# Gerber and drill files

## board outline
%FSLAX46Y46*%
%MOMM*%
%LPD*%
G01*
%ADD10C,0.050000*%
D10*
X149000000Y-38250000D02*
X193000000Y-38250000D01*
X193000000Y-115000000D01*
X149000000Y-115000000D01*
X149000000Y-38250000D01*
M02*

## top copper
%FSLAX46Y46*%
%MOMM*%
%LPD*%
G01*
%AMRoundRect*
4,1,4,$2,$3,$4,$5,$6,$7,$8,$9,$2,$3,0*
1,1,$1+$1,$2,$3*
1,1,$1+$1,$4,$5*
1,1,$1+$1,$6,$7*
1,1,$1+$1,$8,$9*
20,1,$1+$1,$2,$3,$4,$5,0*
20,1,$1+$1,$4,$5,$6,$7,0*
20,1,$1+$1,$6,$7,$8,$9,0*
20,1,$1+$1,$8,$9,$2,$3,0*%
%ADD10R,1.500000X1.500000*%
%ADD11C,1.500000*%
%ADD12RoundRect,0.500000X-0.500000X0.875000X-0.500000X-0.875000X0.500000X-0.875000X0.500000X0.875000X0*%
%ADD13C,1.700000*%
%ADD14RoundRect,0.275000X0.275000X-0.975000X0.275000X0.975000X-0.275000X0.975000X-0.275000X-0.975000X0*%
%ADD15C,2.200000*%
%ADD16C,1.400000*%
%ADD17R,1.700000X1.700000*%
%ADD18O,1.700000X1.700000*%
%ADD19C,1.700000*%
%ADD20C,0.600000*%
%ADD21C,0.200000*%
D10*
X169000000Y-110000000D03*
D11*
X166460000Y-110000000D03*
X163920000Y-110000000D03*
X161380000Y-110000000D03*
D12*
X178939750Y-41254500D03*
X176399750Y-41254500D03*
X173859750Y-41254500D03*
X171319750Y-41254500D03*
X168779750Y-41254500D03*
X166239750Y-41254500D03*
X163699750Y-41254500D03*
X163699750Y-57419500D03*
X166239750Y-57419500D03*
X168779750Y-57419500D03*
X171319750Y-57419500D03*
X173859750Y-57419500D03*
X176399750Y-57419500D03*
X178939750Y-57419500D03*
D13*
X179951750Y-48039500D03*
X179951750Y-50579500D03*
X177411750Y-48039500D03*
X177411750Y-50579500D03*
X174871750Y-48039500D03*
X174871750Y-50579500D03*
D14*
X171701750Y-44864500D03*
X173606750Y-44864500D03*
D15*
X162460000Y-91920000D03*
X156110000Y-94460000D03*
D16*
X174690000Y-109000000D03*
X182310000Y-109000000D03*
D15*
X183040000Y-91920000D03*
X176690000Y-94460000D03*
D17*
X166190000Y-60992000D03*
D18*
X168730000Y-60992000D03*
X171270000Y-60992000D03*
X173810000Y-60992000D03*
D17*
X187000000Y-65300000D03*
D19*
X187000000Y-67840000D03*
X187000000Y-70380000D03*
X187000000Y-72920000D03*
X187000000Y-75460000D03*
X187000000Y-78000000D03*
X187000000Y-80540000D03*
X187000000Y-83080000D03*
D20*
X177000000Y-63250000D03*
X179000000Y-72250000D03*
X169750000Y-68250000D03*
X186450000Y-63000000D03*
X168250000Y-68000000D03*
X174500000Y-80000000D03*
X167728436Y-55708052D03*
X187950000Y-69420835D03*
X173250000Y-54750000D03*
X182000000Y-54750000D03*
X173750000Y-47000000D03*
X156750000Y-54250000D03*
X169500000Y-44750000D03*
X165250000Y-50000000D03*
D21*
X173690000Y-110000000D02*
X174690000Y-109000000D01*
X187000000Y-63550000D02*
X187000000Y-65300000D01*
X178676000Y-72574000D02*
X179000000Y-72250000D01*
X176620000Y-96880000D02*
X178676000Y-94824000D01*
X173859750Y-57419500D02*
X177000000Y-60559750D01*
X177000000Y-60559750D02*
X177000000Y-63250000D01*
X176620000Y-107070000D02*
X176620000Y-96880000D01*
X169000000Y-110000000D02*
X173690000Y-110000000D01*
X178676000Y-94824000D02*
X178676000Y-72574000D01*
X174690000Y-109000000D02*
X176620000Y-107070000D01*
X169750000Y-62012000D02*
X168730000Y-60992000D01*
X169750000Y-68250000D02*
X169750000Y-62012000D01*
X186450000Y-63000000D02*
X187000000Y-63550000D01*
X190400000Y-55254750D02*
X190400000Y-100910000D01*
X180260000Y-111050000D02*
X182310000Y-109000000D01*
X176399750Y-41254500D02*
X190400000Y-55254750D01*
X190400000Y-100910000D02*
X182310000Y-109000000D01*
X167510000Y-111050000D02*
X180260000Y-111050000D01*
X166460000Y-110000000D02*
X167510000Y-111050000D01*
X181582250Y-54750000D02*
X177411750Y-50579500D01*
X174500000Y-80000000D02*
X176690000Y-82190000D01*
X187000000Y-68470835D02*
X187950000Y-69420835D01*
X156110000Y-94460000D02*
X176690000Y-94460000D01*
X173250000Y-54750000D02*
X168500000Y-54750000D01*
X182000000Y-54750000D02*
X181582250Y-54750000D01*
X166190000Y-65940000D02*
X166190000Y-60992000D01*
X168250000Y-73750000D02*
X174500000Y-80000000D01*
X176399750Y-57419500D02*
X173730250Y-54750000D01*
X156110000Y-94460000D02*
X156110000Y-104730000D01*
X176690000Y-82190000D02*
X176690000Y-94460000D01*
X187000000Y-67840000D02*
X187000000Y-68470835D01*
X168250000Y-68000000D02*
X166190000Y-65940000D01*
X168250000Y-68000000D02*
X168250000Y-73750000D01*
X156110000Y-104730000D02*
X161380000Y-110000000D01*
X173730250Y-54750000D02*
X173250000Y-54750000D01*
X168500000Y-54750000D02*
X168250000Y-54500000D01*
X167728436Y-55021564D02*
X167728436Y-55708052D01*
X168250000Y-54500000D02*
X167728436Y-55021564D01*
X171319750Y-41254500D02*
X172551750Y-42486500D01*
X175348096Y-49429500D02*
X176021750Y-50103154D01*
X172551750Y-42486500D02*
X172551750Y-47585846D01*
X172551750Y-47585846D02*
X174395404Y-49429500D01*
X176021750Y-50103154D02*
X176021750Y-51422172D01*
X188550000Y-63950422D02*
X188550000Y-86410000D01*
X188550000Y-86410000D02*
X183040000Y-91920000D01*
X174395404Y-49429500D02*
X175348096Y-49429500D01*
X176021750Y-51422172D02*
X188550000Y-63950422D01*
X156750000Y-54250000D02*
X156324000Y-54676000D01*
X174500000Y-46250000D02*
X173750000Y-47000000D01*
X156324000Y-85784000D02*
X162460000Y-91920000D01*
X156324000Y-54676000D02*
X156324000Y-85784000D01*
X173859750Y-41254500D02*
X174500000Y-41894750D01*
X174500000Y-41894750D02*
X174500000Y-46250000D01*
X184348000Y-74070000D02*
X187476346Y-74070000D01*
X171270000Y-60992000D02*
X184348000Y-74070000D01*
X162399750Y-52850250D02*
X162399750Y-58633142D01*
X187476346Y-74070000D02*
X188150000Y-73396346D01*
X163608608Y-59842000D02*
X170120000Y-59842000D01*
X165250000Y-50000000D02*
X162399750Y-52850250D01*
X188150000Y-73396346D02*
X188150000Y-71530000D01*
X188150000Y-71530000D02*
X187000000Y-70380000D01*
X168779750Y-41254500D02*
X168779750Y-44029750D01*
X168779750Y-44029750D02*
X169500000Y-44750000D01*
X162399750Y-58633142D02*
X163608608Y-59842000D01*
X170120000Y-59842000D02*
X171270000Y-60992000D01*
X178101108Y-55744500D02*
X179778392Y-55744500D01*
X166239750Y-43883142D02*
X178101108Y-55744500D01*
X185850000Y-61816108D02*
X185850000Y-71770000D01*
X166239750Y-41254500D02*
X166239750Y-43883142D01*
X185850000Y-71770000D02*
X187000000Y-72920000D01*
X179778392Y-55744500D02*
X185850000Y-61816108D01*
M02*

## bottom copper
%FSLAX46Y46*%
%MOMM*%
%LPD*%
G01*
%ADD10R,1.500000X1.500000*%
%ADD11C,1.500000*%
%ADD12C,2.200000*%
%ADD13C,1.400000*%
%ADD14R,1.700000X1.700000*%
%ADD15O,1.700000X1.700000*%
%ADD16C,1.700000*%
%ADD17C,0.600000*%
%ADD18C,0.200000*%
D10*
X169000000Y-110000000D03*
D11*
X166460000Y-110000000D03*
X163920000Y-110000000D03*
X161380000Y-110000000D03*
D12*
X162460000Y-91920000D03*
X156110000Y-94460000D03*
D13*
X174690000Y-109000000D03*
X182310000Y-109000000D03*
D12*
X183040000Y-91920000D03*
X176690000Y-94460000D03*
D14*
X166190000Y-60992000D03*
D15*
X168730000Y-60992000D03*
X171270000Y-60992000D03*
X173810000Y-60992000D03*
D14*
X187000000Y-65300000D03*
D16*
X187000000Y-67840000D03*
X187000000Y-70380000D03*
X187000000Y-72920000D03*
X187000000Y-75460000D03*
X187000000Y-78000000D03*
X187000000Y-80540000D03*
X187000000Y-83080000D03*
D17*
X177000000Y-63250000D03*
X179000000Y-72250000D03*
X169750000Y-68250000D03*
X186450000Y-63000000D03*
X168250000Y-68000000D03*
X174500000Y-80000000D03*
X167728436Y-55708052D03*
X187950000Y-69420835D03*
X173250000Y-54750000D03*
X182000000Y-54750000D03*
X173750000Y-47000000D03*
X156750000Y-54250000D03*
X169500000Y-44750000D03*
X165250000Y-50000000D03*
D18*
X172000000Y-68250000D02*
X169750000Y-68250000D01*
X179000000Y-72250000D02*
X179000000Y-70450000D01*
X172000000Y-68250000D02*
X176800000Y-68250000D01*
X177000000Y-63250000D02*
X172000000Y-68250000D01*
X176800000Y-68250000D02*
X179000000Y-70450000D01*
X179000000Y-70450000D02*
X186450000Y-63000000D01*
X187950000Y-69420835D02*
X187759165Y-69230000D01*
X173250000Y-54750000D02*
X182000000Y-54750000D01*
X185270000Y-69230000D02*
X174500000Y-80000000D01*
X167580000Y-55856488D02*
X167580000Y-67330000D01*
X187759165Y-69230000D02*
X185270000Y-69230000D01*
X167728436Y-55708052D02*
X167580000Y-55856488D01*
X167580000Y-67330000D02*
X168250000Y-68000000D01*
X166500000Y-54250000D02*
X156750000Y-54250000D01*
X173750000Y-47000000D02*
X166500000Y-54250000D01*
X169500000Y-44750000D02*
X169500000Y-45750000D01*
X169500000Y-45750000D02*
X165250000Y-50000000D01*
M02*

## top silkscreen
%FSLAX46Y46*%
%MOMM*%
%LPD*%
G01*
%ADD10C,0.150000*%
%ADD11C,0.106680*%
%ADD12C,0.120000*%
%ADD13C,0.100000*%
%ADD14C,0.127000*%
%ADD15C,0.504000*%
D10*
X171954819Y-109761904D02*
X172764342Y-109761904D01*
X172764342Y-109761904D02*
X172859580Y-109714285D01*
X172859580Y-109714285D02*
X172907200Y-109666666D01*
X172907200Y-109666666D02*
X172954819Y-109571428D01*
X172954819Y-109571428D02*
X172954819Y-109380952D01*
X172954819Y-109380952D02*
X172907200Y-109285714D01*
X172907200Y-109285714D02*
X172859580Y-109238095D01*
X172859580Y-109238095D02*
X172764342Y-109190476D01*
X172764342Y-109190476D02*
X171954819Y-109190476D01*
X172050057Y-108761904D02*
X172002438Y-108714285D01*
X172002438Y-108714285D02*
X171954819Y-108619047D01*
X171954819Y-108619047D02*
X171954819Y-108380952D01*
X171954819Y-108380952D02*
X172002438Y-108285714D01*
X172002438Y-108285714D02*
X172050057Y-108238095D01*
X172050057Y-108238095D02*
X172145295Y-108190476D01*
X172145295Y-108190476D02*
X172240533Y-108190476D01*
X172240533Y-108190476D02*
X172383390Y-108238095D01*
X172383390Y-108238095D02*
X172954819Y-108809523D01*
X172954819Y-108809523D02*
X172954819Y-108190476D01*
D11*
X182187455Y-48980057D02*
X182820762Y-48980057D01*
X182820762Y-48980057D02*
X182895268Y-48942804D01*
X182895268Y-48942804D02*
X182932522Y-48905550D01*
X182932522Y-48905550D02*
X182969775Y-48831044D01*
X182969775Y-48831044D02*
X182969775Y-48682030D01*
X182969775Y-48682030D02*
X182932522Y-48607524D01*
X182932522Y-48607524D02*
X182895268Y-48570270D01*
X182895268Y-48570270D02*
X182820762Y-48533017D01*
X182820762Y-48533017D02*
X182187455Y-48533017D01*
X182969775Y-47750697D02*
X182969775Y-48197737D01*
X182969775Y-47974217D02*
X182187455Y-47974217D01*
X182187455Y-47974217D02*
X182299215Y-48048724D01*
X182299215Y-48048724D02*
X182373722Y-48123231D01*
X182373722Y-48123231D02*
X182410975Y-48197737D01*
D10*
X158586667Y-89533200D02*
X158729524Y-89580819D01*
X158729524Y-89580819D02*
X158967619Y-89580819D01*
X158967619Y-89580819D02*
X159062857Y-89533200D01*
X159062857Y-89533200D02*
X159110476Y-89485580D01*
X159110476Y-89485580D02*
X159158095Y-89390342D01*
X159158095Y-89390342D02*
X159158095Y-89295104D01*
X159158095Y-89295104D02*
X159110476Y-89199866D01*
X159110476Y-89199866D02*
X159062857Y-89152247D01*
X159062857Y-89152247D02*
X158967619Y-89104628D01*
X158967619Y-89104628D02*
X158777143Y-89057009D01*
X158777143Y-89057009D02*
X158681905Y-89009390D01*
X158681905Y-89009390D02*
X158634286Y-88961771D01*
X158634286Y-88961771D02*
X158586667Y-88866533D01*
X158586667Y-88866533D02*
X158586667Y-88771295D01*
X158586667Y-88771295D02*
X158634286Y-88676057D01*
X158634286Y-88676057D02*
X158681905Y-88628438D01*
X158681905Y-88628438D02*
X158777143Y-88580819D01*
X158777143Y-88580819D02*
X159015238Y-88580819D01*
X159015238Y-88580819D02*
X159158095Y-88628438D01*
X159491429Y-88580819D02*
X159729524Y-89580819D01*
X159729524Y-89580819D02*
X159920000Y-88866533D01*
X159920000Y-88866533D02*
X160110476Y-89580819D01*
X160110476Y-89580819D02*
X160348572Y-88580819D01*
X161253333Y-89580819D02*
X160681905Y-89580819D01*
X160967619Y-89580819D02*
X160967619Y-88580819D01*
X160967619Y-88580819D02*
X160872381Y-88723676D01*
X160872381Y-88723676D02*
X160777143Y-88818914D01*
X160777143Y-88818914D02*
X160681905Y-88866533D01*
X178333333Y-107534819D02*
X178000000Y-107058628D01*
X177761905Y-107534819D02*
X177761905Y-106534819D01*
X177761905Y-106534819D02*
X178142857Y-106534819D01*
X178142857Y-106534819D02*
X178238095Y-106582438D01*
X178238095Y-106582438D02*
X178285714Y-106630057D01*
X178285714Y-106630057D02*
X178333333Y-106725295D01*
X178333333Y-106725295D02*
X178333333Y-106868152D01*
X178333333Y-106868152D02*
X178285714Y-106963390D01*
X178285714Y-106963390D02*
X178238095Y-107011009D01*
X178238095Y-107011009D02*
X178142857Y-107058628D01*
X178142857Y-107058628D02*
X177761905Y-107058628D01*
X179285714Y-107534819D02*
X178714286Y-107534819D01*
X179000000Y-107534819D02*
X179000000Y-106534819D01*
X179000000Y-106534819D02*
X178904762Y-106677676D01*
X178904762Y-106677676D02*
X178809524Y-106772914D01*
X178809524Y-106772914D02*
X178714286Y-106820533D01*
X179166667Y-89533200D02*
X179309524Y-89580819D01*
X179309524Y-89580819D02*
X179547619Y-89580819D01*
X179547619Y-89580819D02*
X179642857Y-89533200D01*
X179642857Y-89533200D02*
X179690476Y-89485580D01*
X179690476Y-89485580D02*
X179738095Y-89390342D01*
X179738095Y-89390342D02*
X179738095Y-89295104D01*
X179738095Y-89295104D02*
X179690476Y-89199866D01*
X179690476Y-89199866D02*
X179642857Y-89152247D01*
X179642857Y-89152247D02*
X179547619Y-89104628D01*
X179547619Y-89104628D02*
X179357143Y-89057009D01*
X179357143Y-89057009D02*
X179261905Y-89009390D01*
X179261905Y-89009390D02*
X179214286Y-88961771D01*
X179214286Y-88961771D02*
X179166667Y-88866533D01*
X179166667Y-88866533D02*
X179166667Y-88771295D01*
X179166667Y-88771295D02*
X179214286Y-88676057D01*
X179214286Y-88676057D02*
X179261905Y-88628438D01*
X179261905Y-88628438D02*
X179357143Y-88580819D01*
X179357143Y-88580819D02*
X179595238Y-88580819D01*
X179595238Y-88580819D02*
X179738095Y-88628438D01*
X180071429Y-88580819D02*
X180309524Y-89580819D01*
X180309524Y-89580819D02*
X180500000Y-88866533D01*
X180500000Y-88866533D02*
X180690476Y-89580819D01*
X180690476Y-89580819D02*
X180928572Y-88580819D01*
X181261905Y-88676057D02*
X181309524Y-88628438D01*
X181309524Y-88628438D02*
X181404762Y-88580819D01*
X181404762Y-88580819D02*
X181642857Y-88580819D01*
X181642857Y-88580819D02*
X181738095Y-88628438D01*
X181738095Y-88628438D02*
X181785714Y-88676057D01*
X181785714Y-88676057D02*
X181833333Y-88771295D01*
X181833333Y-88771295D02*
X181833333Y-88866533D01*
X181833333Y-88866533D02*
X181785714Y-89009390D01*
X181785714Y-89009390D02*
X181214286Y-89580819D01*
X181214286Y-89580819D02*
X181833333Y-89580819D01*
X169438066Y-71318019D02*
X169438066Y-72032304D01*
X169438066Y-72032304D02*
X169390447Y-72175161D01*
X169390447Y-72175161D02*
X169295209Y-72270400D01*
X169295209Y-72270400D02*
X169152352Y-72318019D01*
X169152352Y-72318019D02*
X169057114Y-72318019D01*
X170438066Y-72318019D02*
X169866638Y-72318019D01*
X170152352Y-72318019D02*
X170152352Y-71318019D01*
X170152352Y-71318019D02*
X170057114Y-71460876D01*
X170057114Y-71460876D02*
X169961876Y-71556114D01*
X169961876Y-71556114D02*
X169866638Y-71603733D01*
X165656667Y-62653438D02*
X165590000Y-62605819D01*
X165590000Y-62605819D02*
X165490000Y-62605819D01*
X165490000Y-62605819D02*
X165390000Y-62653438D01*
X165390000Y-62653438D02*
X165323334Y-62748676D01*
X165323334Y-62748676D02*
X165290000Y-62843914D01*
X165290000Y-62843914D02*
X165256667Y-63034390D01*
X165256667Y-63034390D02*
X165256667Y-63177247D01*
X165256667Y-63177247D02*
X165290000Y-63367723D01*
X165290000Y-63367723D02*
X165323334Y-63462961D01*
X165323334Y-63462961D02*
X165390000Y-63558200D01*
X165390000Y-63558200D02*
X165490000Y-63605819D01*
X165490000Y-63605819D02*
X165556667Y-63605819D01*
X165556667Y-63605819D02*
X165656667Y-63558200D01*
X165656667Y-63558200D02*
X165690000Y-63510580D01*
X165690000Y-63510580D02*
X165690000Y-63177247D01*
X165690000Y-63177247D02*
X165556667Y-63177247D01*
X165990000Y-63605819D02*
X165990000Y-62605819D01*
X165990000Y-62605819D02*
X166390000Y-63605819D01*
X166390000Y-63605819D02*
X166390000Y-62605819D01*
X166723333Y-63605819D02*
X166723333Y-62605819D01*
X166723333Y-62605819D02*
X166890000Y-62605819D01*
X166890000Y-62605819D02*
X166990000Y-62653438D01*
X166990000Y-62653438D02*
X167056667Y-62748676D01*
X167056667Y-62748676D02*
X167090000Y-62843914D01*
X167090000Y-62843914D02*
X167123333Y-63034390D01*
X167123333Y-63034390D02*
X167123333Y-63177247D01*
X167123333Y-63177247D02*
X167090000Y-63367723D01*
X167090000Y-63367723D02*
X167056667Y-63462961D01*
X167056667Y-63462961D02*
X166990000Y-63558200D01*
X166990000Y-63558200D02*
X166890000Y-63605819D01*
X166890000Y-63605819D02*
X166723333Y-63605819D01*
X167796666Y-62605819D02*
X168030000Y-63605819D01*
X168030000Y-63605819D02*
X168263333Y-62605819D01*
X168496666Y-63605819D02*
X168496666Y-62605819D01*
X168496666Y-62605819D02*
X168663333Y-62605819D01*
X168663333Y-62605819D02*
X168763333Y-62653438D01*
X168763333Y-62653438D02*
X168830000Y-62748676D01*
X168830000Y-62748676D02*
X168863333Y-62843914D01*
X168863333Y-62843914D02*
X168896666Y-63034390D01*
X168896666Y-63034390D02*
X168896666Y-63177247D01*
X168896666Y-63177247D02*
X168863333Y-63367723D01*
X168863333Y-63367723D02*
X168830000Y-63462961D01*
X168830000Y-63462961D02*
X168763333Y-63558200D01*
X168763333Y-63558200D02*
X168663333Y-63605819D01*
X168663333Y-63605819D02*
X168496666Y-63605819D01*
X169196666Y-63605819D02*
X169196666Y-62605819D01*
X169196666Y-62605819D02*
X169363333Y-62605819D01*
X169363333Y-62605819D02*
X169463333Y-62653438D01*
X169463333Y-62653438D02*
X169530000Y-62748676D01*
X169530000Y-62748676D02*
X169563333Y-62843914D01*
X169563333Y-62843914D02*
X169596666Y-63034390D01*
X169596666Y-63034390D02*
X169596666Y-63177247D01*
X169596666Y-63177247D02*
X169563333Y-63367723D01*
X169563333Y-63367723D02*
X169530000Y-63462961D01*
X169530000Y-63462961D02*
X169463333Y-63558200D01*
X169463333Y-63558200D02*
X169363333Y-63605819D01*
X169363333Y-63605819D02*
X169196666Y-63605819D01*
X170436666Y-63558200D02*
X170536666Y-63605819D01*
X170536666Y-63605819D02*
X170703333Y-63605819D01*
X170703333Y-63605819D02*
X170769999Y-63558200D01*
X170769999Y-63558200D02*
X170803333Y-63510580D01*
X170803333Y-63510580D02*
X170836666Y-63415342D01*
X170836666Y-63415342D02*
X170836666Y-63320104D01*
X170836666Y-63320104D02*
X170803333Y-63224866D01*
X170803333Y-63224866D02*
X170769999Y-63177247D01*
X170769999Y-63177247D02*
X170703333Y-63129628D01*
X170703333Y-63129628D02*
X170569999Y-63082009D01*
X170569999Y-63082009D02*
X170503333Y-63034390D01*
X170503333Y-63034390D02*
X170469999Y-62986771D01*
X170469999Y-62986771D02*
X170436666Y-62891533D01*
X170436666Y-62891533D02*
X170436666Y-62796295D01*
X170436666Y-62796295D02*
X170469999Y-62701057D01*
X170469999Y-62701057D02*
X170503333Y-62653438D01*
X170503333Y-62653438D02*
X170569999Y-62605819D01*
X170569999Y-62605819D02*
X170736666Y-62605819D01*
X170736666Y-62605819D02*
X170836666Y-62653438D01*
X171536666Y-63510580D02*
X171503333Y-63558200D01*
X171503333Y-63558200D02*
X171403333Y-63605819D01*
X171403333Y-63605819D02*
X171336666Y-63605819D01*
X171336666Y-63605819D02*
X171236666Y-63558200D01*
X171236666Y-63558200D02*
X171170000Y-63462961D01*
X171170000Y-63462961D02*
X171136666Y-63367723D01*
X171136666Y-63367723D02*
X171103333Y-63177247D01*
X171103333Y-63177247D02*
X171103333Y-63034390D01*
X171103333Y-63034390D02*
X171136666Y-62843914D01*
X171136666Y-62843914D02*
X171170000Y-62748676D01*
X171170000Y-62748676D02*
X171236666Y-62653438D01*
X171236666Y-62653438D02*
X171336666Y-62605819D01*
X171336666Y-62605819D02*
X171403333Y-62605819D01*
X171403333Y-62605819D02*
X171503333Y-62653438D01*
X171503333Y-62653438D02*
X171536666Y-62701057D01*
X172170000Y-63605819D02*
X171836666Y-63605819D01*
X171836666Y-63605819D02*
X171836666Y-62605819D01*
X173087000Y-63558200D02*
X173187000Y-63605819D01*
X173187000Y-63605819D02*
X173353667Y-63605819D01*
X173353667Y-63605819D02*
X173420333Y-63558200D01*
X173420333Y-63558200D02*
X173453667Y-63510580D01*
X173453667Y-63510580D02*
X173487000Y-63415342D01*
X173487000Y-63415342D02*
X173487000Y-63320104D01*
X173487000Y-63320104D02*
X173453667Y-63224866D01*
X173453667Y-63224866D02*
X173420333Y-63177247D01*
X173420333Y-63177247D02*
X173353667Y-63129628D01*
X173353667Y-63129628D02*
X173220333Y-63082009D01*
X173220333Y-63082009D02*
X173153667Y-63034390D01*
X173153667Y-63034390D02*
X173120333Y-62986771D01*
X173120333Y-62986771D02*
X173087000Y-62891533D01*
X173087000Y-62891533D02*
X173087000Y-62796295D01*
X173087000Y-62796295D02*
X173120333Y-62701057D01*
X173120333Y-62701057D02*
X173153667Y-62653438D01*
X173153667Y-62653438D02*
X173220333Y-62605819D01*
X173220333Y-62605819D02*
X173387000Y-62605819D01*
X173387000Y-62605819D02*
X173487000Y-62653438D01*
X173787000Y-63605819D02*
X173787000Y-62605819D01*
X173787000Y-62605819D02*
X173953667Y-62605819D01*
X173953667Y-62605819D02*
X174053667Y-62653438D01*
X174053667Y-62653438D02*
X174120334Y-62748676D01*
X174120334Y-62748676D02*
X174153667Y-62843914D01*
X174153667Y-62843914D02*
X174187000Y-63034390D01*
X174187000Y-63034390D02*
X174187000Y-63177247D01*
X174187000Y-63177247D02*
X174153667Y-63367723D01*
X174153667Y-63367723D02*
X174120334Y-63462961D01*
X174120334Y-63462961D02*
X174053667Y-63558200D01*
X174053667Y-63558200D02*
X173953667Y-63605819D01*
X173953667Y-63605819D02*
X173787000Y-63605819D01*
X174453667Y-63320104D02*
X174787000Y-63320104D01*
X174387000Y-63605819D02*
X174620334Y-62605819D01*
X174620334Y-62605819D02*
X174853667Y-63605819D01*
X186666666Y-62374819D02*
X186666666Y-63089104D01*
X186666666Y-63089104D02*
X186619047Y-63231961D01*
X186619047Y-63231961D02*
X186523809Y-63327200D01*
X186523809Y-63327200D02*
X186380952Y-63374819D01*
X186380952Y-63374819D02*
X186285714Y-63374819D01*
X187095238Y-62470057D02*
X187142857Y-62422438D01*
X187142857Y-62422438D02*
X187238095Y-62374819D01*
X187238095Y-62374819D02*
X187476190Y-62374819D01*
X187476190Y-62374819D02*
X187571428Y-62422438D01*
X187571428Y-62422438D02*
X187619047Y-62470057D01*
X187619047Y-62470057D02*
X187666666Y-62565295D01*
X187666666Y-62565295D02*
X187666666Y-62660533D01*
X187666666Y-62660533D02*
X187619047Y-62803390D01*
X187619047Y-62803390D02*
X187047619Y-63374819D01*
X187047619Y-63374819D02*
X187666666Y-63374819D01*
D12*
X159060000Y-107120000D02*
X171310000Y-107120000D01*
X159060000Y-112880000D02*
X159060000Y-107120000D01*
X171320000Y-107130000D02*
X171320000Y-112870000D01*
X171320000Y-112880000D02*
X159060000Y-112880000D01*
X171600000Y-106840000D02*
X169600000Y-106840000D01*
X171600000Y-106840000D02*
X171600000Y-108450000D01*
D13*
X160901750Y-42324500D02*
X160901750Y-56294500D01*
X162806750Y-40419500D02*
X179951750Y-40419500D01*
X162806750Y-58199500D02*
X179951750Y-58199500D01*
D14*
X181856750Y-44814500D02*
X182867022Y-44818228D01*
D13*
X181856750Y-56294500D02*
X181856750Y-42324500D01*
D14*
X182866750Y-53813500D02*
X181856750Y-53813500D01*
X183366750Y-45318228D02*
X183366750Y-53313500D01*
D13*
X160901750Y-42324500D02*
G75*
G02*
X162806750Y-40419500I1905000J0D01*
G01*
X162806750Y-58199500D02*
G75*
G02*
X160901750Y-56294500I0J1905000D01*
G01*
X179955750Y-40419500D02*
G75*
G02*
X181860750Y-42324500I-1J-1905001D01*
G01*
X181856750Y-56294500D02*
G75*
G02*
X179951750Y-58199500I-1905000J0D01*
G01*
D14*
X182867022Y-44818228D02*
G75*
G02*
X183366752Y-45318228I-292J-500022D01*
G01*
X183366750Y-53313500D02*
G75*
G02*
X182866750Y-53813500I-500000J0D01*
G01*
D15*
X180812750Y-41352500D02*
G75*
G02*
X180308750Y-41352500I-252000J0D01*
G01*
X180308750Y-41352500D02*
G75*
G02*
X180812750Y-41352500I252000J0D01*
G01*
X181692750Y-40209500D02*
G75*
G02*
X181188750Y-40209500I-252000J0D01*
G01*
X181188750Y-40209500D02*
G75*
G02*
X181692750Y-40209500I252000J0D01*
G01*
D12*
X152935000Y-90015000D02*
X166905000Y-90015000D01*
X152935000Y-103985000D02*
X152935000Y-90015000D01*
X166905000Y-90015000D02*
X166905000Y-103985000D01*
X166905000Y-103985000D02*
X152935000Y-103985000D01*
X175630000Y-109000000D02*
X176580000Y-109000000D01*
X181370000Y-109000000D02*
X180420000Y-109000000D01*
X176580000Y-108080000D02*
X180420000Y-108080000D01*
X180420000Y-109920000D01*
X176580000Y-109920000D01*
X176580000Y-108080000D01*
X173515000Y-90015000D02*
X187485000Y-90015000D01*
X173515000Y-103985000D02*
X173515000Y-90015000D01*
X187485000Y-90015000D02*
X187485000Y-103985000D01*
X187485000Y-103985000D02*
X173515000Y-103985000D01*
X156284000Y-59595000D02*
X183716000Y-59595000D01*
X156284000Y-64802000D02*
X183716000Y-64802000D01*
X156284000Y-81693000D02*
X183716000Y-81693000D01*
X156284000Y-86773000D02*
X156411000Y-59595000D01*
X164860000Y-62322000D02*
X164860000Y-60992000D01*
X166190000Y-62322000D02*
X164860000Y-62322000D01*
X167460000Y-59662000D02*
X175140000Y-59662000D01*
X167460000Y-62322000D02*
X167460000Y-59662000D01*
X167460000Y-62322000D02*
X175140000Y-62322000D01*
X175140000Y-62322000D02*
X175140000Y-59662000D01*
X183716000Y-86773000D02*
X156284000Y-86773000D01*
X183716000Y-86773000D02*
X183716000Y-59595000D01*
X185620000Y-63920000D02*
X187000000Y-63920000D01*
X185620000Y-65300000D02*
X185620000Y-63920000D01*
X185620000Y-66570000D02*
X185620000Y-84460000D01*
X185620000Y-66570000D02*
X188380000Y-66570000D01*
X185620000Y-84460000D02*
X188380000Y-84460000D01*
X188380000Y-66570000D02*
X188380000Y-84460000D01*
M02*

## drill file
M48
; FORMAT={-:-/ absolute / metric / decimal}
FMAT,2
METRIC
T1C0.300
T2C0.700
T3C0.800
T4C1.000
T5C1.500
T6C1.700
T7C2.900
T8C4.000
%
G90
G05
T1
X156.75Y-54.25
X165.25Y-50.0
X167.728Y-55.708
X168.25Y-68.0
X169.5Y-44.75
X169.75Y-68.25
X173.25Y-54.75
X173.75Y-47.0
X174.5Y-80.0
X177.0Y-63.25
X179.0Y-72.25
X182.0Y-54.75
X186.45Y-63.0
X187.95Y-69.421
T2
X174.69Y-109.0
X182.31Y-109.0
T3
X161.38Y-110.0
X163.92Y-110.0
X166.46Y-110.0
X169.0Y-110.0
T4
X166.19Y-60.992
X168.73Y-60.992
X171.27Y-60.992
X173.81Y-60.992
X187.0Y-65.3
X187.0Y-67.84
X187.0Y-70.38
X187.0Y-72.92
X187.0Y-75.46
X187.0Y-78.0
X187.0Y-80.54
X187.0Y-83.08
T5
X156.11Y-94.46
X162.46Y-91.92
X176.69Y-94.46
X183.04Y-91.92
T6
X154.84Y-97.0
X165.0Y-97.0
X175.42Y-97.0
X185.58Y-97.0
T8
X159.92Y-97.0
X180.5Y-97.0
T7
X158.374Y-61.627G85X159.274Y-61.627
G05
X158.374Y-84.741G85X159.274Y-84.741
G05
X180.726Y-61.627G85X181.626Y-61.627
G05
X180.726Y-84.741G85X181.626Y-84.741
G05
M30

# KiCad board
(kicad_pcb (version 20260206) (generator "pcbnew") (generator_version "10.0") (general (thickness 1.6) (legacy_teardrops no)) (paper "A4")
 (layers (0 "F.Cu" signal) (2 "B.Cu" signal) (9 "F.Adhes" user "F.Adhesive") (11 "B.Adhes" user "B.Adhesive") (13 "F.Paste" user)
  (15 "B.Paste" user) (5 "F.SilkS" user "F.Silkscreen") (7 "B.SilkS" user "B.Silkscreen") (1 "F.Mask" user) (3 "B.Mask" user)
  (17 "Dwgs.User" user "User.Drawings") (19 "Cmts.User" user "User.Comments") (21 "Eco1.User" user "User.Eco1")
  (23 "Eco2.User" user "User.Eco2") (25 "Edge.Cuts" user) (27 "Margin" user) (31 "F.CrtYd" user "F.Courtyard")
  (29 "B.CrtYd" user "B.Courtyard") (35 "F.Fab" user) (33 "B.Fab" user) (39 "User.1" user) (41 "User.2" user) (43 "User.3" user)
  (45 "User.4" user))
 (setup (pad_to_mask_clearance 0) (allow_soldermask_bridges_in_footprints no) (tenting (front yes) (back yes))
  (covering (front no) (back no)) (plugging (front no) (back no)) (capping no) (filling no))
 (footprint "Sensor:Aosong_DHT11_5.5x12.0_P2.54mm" (layer "F.Cu") (at 169 110 -90)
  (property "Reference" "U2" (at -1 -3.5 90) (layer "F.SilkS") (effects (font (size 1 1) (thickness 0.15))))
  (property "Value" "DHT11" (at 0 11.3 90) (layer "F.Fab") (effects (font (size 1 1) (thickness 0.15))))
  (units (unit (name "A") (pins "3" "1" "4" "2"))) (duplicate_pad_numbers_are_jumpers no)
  (fp_line (start -2.88 9.94) (end -2.88 -2.31) (stroke (width 0.12) (type solid)) (layer "F.SilkS"))
  (fp_line (start 2.88 9.94) (end -2.88 9.94) (stroke (width 0.12) (type solid)) (layer "F.SilkS"))
  (fp_line (start -2.87 -2.32) (end 2.87 -2.32) (stroke (width 0.12) (type solid)) (layer "F.SilkS"))
  (fp_line (start 2.88 -2.32) (end 2.88 9.94) (stroke (width 0.12) (type solid)) (layer "F.SilkS"))
  (fp_line (start -3.16 -2.6) (end -3.16 -0.6) (stroke (width 0.12) (type solid)) (layer "F.SilkS"))
  (fp_line (start -3.16 -2.6) (end -1.55 -2.6) (stroke (width 0.12) (type solid)) (layer "F.SilkS"))
  (pad "1" thru_hole rect (at 0 0 270) (size 1.5 1.5) (drill 0.8) (layers "*.Cu" "*.Mask") (remove_unused_layers no) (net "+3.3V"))
  (pad "2" thru_hole circle (at 0 2.54 270) (size 1.5 1.5) (drill 0.8) (layers "*.Cu" "*.Mask") (remove_unused_layers no)
   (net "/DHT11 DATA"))
  (pad "3" thru_hole circle (at 0 5.08 270) (size 1.5 1.5) (drill 0.8) (layers "*.Cu" "*.Mask") (remove_unused_layers no)
   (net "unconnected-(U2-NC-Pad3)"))
  (pad "4" thru_hole circle (at 0 7.62 270) (size 1.5 1.5) (drill 0.8) (layers "*.Cu" "*.Mask") (remove_unused_layers no) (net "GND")))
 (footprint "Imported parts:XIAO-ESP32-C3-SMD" (layer "F.Cu") (at 160.81975 40.4195 -90)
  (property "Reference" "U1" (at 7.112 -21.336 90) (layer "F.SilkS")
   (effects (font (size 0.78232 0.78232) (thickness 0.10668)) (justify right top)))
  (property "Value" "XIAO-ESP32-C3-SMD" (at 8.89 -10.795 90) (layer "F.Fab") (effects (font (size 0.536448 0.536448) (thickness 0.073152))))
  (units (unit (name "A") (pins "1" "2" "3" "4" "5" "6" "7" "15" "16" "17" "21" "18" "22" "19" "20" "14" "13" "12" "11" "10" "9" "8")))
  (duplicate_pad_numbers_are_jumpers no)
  (fp_line (start 1.905 -0.082) (end 15.875 -0.082) (stroke (width 0.1) (type solid)) (layer "F.SilkS"))
  (fp_line (start 0 -1.987) (end 0 -19.132) (stroke (width 0.1) (type solid)) (layer "F.SilkS"))
  (fp_line (start 17.78 -1.987) (end 17.78 -19.132) (stroke (width 0.1) (type solid)) (layer "F.SilkS"))
  (fp_line (start 4.395 -21.037) (end 4.398728 -22.047272) (stroke (width 0.127) (type solid)) (layer "F.SilkS"))
  (fp_line (start 15.875 -21.037) (end 1.905 -21.037) (stroke (width 0.1) (type solid)) (layer "F.SilkS"))
  (fp_line (start 13.394 -22.047) (end 13.394 -21.037) (stroke (width 0.127) (type solid)) (layer "F.SilkS"))
  (fp_line (start 4.898728 -22.547) (end 12.894 -22.547) (stroke (width 0.127) (type solid)) (layer "F.SilkS"))
  (fp_arc (start 1.905 -0.082) (mid 0.557962 -0.639962) (end 0 -1.987) (stroke (width 0.1) (type solid)) (layer "F.SilkS"))
  (fp_arc (start 17.78 -1.987) (mid 17.222038 -0.639962) (end 15.875 -0.082) (stroke (width 0.1) (type solid)) (layer "F.SilkS"))
  (fp_arc (start 0 -19.136) (mid 0.557962 -20.483038) (end 1.905 -21.041) (stroke (width 0.1) (type solid)) (layer "F.SilkS"))
  (fp_arc (start 15.875 -21.037) (mid 17.222038 -20.479038) (end 17.78 -19.132) (stroke (width 0.1) (type solid)) (layer "F.SilkS"))
  (fp_arc (start 4.398728 -22.047272) (mid 4.545272 -22.40064) (end 4.898728 -22.547) (stroke (width 0.127) (type default))
   (layer "F.SilkS"))
  (fp_arc (start 12.894 -22.547) (mid 13.247553 -22.400553) (end 13.394 -22.047) (stroke (width 0.127) (type default)) (layer "F.SilkS"))
  (fp_circle (center 0.933 -19.741) (end 0.933 -19.995) (stroke (width 0.5) (type solid)) (fill yes) (layer "F.SilkS"))
  (fp_circle (center -0.21 -20.621) (end -0.21 -20.875) (stroke (width 0.5) (type solid)) (fill yes) (layer "F.SilkS"))
  (pad "1" smd roundrect (at 0.835 -18.12 270) (size 2.75 2) (layers "F.Cu" "F.Mask" "F.Paste") (roundrect_rratio 0.25)
   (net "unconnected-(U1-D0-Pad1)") (solder_mask_margin 0.0508) (thermal_bridge_angle 45))
  (pad "2" smd roundrect (at 0.835 -15.58 270) (size 2.75 2) (layers "F.Cu" "F.Mask" "F.Paste") (roundrect_rratio 0.25) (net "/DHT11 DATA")
   (solder_mask_margin 0.0508) (thermal_bridge_angle 45))
  (pad "3" smd roundrect (at 0.835 -13.04 270) (size 2.75 2) (layers "F.Cu" "F.Mask" "F.Paste") (roundrect_rratio 0.25) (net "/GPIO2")
   (solder_mask_margin 0.0508) (thermal_bridge_angle 45))
  (pad "4" smd roundrect (at 0.835 -10.5 270) (size 2.75 2) (layers "F.Cu" "F.Mask" "F.Paste") (roundrect_rratio 0.25) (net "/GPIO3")
   (solder_mask_margin 0.0508) (thermal_bridge_angle 45))
  (pad "5" smd roundrect (at 0.835 -7.96 270) (size 2.75 2) (layers "F.Cu" "F.Mask" "F.Paste") (roundrect_rratio 0.25) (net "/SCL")
   (solder_mask_margin 0.0508) (thermal_bridge_angle 45))
  (pad "6" smd roundrect (at 0.835 -5.42 270) (size 2.75 2) (layers "F.Cu" "F.Mask" "F.Paste") (roundrect_rratio 0.25) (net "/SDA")
   (solder_mask_margin 0.0508) (thermal_bridge_angle 45))
  (pad "7" smd roundrect (at 0.835 -2.88 270) (size 2.75 2) (layers "F.Cu" "F.Mask" "F.Paste") (roundrect_rratio 0.25)
   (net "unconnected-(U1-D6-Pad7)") (solder_mask_margin 0.0508) (thermal_bridge_angle 45))
  (pad "8" smd roundrect (at 17 -2.88 270) (size 2.75 2) (layers "F.Cu" "F.Mask" "F.Paste") (roundrect_rratio 0.25)
   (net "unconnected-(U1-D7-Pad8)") (solder_mask_margin 0.0508) (thermal_bridge_angle 45))
  (pad "9" smd roundrect (at 17 -5.42 270) (size 2.75 2) (layers "F.Cu" "F.Mask" "F.Paste") (roundrect_rratio 0.25)
   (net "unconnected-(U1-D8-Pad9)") (solder_mask_margin 0.0508) (thermal_bridge_angle 45))
  (pad "10" smd roundrect (at 17 -7.96 270) (size 2.75 2) (layers "F.Cu" "F.Mask" "F.Paste") (roundrect_rratio 0.25)
   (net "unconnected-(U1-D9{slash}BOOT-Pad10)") (solder_mask_margin 0.0508) (thermal_bridge_angle 45))
  (pad "11" smd roundrect (at 17 -10.5 270) (size 2.75 2) (layers "F.Cu" "F.Mask" "F.Paste") (roundrect_rratio 0.25)
   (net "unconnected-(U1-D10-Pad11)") (solder_mask_margin 0.0508) (thermal_bridge_angle 45))
  (pad "12" smd roundrect (at 17 -13.04 270) (size 2.75 2) (layers "F.Cu" "F.Mask" "F.Paste") (roundrect_rratio 0.25) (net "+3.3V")
   (solder_mask_margin 0.0508) (thermal_bridge_angle 45))
  (pad "13" smd roundrect (at 17 -15.58 270) (size 2.75 2) (layers "F.Cu" "F.Mask" "F.Paste") (roundrect_rratio 0.25) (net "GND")
   (solder_mask_margin 0.0508) (thermal_bridge_angle 45))
  (pad "14" smd roundrect (at 17 -18.12 270) (size 2.75 2) (layers "F.Cu" "F.Mask" "F.Paste") (roundrect_rratio 0.25) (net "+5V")
   (solder_mask_margin 0.0508) (thermal_bridge_angle 45))
  (pad "15" smd circle (at 7.62 -19.132 270) (size 1.7 1.7) (layers "F.Cu" "F.Mask" "F.Paste") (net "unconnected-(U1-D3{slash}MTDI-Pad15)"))
  (pad "16" smd circle (at 10.16 -19.132 270) (size 1.7 1.7) (layers "F.Cu" "F.Mask" "F.Paste") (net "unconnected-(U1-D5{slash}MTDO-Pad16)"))
  (pad "17" smd circle (at 7.62 -16.592 270) (size 1.7 1.7) (layers "F.Cu" "F.Mask" "F.Paste") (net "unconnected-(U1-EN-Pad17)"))
  (pad "18" smd circle (at 10.16 -16.592 270) (size 1.7 1.7) (layers "F.Cu" "F.Mask" "F.Paste") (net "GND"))
  (pad "19" smd circle (at 7.62 -14.052 270) (size 1.7 1.7) (layers "F.Cu" "F.Mask" "F.Paste") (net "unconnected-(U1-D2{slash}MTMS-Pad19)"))
  (pad "20" smd circle (at 10.16 -14.052 270) (size 1.7 1.7) (layers "F.Cu" "F.Mask" "F.Paste") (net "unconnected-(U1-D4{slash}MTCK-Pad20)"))
  (pad "21" smd roundrect (at 4.445 -10.882 90) (size 2.5 1.1) (layers "F.Cu" "F.Mask" "F.Paste") (roundrect_rratio 0.25)
   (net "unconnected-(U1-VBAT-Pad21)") (thermal_bridge_angle 45))
  (pad "22" smd roundrect (at 4.445 -12.787 90) (size 2.5 1.1) (layers "F.Cu" "F.Mask" "F.Paste") (roundrect_rratio 0.25)
   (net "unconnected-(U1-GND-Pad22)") (thermal_bridge_angle 45)))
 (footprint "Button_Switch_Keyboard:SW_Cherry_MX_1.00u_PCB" (layer "F.Cu") (at 162.46 91.92)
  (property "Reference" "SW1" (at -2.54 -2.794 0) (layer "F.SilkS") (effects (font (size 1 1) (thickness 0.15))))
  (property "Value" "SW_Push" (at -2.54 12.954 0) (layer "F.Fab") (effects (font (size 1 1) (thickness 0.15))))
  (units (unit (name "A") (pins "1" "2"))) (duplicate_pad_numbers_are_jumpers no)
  (fp_line (start -9.525 -1.905) (end 4.445 -1.905) (stroke (width 0.12) (type solid)) (layer "F.SilkS"))
  (fp_line (start -9.525 12.065) (end -9.525 -1.905) (stroke (width 0.12) (type solid)) (layer "F.SilkS"))
  (fp_line (start 4.445 -1.905) (end 4.445 12.065) (stroke (width 0.12) (type solid)) (layer "F.SilkS"))
  (fp_line (start 4.445 12.065) (end -9.525 12.065) (stroke (width 0.12) (type solid)) (layer "F.SilkS"))
  (pad "" np_thru_hole circle (at -7.62 5.08) (size 1.7 1.7) (drill 1.7) (layers "*.Cu" "*.Mask"))
  (pad "" np_thru_hole circle (at -2.54 5.08) (size 4 4) (drill 4) (layers "*.Cu" "*.Mask"))
  (pad "" np_thru_hole circle (at 2.54 5.08) (size 1.7 1.7) (drill 1.7) (layers "*.Cu" "*.Mask"))
  (pad "1" thru_hole circle (at 0 0) (size 2.2 2.2) (drill 1.5) (layers "*.Cu" "*.Mask") (remove_unused_layers no) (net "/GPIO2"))
  (pad "2" thru_hole circle (at -6.35 2.54) (size 2.2 2.2) (drill 1.5) (layers "*.Cu" "*.Mask") (remove_unused_layers no) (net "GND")))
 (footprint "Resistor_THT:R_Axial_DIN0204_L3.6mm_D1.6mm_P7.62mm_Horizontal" (layer "F.Cu") (at 174.69 109)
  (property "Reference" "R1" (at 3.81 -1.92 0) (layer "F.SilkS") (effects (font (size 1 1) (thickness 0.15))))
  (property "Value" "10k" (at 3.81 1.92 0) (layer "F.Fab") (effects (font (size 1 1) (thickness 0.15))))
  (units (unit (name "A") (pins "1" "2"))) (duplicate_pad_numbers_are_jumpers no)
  (fp_line (start 0.94 0) (end 1.89 0) (stroke (width 0.12) (type solid)) (layer "F.SilkS"))
  (fp_line (start 6.68 0) (end 5.73 0) (stroke (width 0.12) (type solid)) (layer "F.SilkS"))
  (fp_rect (start 1.89 -0.92) (end 5.73 0.92) (stroke (width 0.12) (type solid)) (fill no) (layer "F.SilkS"))
  (pad "1" thru_hole circle (at 0 0) (size 1.4 1.4) (drill 0.7) (layers "*.Cu" "*.Mask") (remove_unused_layers no) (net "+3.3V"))
  (pad "2" thru_hole circle (at 7.62 0) (size 1.4 1.4) (drill 0.7) (layers "*.Cu" "*.Mask") (remove_unused_layers no) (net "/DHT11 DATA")))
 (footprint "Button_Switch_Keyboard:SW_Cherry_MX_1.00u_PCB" (layer "F.Cu") (at 183.04 91.92)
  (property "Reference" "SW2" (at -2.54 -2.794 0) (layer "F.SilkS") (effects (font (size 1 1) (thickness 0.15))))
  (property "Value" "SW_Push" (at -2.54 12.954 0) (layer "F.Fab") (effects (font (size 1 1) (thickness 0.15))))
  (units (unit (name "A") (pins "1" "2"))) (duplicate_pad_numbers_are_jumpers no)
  (fp_line (start -9.525 -1.905) (end 4.445 -1.905) (stroke (width 0.12) (type solid)) (layer "F.SilkS"))
  (fp_line (start -9.525 12.065) (end -9.525 -1.905) (stroke (width 0.12) (type solid)) (layer "F.SilkS"))
  (fp_line (start 4.445 -1.905) (end 4.445 12.065) (stroke (width 0.12) (type solid)) (layer "F.SilkS"))
  (fp_line (start 4.445 12.065) (end -9.525 12.065) (stroke (width 0.12) (type solid)) (layer "F.SilkS"))
  (pad "" np_thru_hole circle (at -7.62 5.08) (size 1.7 1.7) (drill 1.7) (layers "*.Cu" "*.Mask"))
  (pad "" np_thru_hole circle (at -2.54 5.08) (size 4 4) (drill 4) (layers "*.Cu" "*.Mask"))
  (pad "" np_thru_hole circle (at 2.54 5.08) (size 1.7 1.7) (drill 1.7) (layers "*.Cu" "*.Mask"))
  (pad "1" thru_hole circle (at 0 0) (size 2.2 2.2) (drill 1.5) (layers "*.Cu" "*.Mask") (remove_unused_layers no) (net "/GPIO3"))
  (pad "2" thru_hole circle (at -6.35 2.54) (size 2.2 2.2) (drill 1.5) (layers "*.Cu" "*.Mask") (remove_unused_layers no) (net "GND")))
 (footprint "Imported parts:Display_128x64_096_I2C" (layer "F.Cu") (at 170 60.992)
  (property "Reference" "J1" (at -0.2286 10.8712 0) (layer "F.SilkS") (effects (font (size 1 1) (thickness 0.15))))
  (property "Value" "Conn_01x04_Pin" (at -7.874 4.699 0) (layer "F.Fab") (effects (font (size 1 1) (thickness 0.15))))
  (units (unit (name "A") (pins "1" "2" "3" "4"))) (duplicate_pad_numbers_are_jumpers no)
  (fp_line (start -13.716 -1.397) (end 13.716 -1.397) (stroke (width 0.12) (type solid)) (layer "F.SilkS"))
  (fp_line (start -13.716 3.81) (end 13.716 3.81) (stroke (width 0.12) (type solid)) (layer "F.SilkS"))
  (fp_line (start -13.716 20.701) (end 13.716 20.701) (stroke (width 0.12) (type solid)) (layer "F.SilkS"))
  (fp_line (start -13.716 25.781) (end -13.589 -1.397) (stroke (width 0.12) (type solid)) (layer "F.SilkS"))
  (fp_line (start -5.14 1.33) (end -5.14 0) (stroke (width 0.12) (type solid)) (layer "F.SilkS"))
  (fp_line (start -3.81 1.33) (end -5.14 1.33) (stroke (width 0.12) (type solid)) (layer "F.SilkS"))
  (fp_line (start -2.54 -1.33) (end 5.14 -1.33) (stroke (width 0.12) (type solid)) (layer "F.SilkS"))
  (fp_line (start -2.54 1.33) (end -2.54 -1.33) (stroke (width 0.12) (type solid)) (layer "F.SilkS"))
  (fp_line (start -2.54 1.33) (end 5.14 1.33) (stroke (width 0.12) (type solid)) (layer "F.SilkS"))
  (fp_line (start 5.14 1.33) (end 5.14 -1.33) (stroke (width 0.12) (type solid)) (layer "F.SilkS"))
  (fp_line (start 13.716 25.781) (end -13.716 25.781) (stroke (width 0.12) (type solid)) (layer "F.SilkS"))
  (fp_line (start 13.716 25.781) (end 13.716 -1.397) (stroke (width 0.12) (type solid)) (layer "F.SilkS"))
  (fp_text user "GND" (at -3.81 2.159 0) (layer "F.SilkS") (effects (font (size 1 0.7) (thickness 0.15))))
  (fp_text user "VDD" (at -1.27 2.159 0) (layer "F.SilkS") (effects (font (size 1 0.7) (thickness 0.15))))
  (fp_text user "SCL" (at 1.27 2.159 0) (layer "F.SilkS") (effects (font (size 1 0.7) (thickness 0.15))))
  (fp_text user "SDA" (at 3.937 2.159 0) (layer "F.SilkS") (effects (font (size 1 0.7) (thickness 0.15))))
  (pad "" np_thru_hole oval (at -11.176 0.635) (size 3.8 2.9) (drill oval 3.8 2.9) (layers "*.Cu" "*.Mask"))
  (pad "" np_thru_hole oval (at -11.176 23.749) (size 3.8 2.9) (drill oval 3.8 2.9) (layers "*.Cu" "*.Mask"))
  (pad "" np_thru_hole oval (at 11.176 0.635) (size 3.8 2.9) (drill oval 3.8 2.9) (layers "*.Cu" "*.Mask"))
  (pad "" np_thru_hole oval (at 11.176 23.749) (size 3.8 2.9) (drill oval 3.8 2.9) (layers "*.Cu" "*.Mask"))
  (pad "1" thru_hole rect (at -3.81 0 90) (size 1.7 1.7) (drill 1) (layers "*.Cu" "*.Mask") (remove_unused_layers no) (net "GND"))
  (pad "2" thru_hole oval (at -1.27 0 90) (size 1.7 1.7) (drill 1) (layers "*.Cu" "*.Mask") (remove_unused_layers no) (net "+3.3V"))
  (pad "3" thru_hole oval (at 1.27 0 90) (size 1.7 1.7) (drill 1) (layers "*.Cu" "*.Mask") (remove_unused_layers no) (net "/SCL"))
  (pad "4" thru_hole oval (at 3.81 0 90) (size 1.7 1.7) (drill 1) (layers "*.Cu" "*.Mask") (remove_unused_layers no) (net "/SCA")))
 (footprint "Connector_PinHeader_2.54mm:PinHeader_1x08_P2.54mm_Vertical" (layer "F.Cu") (at 187 65.3)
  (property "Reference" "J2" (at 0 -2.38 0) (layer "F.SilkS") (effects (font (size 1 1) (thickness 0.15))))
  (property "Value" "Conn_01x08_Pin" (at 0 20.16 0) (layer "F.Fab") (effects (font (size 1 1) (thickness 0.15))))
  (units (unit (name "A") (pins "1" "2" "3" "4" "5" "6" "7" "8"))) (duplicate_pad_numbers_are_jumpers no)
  (fp_line (start -1.38 -1.38) (end 0 -1.38) (stroke (width 0.12) (type solid)) (layer "F.SilkS"))
  (fp_line (start -1.38 0) (end -1.38 -1.38) (stroke (width 0.12) (type solid)) (layer "F.SilkS"))
  (fp_line (start -1.38 1.27) (end -1.38 19.16) (stroke (width 0.12) (type solid)) (layer "F.SilkS"))
  (fp_line (start -1.38 1.27) (end 1.38 1.27) (stroke (width 0.12) (type solid)) (layer "F.SilkS"))
  (fp_line (start -1.38 19.16) (end 1.38 19.16) (stroke (width 0.12) (type solid)) (layer "F.SilkS"))
  (fp_line (start 1.38 1.27) (end 1.38 19.16) (stroke (width 0.12) (type solid)) (layer "F.SilkS"))
  (pad "1" thru_hole rect (at 0 0) (size 1.7 1.7) (drill 1) (layers "*.Cu" "*.Mask") (remove_unused_layers no) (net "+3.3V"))
  (pad "2" thru_hole circle (at 0 2.54) (size 1.7 1.7) (drill 1) (layers "*.Cu" "*.Mask") (remove_unused_layers no) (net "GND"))
  (pad "3" thru_hole circle (at 0 5.08) (size 1.7 1.7) (drill 1) (layers "*.Cu" "*.Mask") (remove_unused_layers no) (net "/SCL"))
  (pad "4" thru_hole circle (at 0 7.62) (size 1.7 1.7) (drill 1) (layers "*.Cu" "*.Mask") (remove_unused_layers no) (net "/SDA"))
  (pad "5" thru_hole circle (at 0 10.16) (size 1.7 1.7) (drill 1) (layers "*.Cu" "*.Mask") (remove_unused_layers no)
   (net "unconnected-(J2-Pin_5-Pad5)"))
  (pad "6" thru_hole circle (at 0 12.7) (size 1.7 1.7) (drill 1) (layers "*.Cu" "*.Mask") (remove_unused_layers no)
   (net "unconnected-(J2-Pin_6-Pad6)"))
  (pad "7" thru_hole circle (at 0 15.24) (size 1.7 1.7) (drill 1) (layers "*.Cu" "*.Mask") (remove_unused_layers no)
   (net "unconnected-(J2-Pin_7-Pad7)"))
  (pad "8" thru_hole circle (at 0 17.78) (size 1.7 1.7) (drill 1) (layers "*.Cu" "*.Mask") (remove_unused_layers no)
   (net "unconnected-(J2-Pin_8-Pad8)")))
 (gr_rect (start 149 38.25) (end 193 115) (stroke (width 0.05) (type default)) (fill no) (layer "Edge.Cuts"))
 (segment (start 173.69 110) (end 174.69 109) (width 0.2) (layer "F.Cu") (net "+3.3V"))
 (segment (start 187 63.55) (end 187 65.3) (width 0.2) (layer "F.Cu") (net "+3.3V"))
 (segment (start 178.676 72.574) (end 179 72.25) (width 0.2) (layer "F.Cu") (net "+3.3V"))
 (segment (start 176.62 96.88) (end 178.676 94.824) (width 0.2) (layer "F.Cu") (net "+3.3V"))
 (segment (start 173.85975 57.4195) (end 177 60.55975) (width 0.2) (layer "F.Cu") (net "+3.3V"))
 (segment (start 177 60.55975) (end 177 63.25) (width 0.2) (layer "F.Cu") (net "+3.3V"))
 (segment (start 176.62 107.07) (end 176.62 96.88) (width 0.2) (layer "F.Cu") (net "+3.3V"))
 (segment (start 169 110) (end 173.69 110) (width 0.2) (layer "F.Cu") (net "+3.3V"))
 (segment (start 178.676 94.824) (end 178.676 72.574) (width 0.2) (layer "F.Cu") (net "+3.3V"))
 (segment (start 174.69 109) (end 176.62 107.07) (width 0.2) (layer "F.Cu") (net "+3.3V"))
 (segment (start 169.75 62.012) (end 168.73 60.992) (width 0.2) (layer "F.Cu") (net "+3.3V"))
 (segment (start 169.75 68.25) (end 169.75 62.012) (width 0.2) (layer "F.Cu") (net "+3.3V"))
 (segment (start 186.45 63) (end 187 63.55) (width 0.2) (layer "F.Cu") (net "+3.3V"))
 (via (at 177 63.25) (size 0.6) (drill 0.3) (layers "F.Cu" "B.Cu") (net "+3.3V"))
 (via (at 179 72.25) (size 0.6) (drill 0.3) (layers "F.Cu" "B.Cu") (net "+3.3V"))
 (via (at 169.75 68.25) (size 0.6) (drill 0.3) (layers "F.Cu" "B.Cu") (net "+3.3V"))
 (via (at 186.45 63) (size 0.6) (drill 0.3) (layers "F.Cu" "B.Cu") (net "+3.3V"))
 (segment (start 172 68.25) (end 169.75 68.25) (width 0.2) (layer "B.Cu") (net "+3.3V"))
 (segment (start 179 72.25) (end 179 70.45) (width 0.2) (layer "B.Cu") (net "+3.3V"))
 (segment (start 172 68.25) (end 176.8 68.25) (width 0.2) (layer "B.Cu") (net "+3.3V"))
 (segment (start 177 63.25) (end 172 68.25) (width 0.2) (layer "B.Cu") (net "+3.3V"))
 (segment (start 176.8 68.25) (end 179 70.45) (width 0.2) (layer "B.Cu") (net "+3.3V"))
 (segment (start 179 70.45) (end 186.45 63) (width 0.2) (layer "B.Cu") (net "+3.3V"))
 (segment (start 190.4 55.25475) (end 190.4 100.91) (width 0.2) (layer "F.Cu") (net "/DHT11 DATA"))
 (segment (start 180.26 111.05) (end 182.31 109) (width 0.2) (layer "F.Cu") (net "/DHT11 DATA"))
 (segment (start 176.39975 41.2545) (end 190.4 55.25475) (width 0.2) (layer "F.Cu") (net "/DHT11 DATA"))
 (segment (start 190.4 100.91) (end 182.31 109) (width 0.2) (layer "F.Cu") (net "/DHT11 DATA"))
 (segment (start 167.51 111.05) (end 180.26 111.05) (width 0.2) (layer "F.Cu") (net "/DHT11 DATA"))
 (segment (start 166.46 110) (end 167.51 111.05) (width 0.2) (layer "F.Cu") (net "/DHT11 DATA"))
 (segment (start 181.58225 54.75) (end 177.41175 50.5795) (width 0.2) (layer "F.Cu") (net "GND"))
 (segment (start 174.5 80) (end 176.69 82.19) (width 0.2) (layer "F.Cu") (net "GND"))
 (segment (start 187 68.470835) (end 187.95 69.420835) (width 0.2) (layer "F.Cu") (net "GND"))
 (segment (start 156.11 94.46) (end 176.69 94.46) (width 0.2) (layer "F.Cu") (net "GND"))
 (segment (start 173.25 54.75) (end 168.5 54.75) (width 0.2) (layer "F.Cu") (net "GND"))
 (segment (start 182 54.75) (end 181.58225 54.75) (width 0.2) (layer "F.Cu") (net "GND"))
 (segment (start 166.19 65.94) (end 166.19 60.992) (width 0.2) (layer "F.Cu") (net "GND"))
 (segment (start 168.25 73.75) (end 174.5 80) (width 0.2) (layer "F.Cu") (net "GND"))
 (segment (start 176.39975 57.4195) (end 173.73025 54.75) (width 0.2) (layer "F.Cu") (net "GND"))
 (segment (start 156.11 94.46) (end 156.11 104.73) (width 0.2) (layer "F.Cu") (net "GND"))
 (segment (start 176.69 82.19) (end 176.69 94.46) (width 0.2) (layer "F.Cu") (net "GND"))
 (segment (start 187 67.84) (end 187 68.470835) (width 0.2) (layer "F.Cu") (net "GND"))
 (segment (start 168.25 68) (end 166.19 65.94) (width 0.2) (layer "F.Cu") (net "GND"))
 (segment (start 168.25 68) (end 168.25 73.75) (width 0.2) (layer "F.Cu") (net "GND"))
 (segment (start 156.11 104.73) (end 161.38 110) (width 0.2) (layer "F.Cu") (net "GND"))
 (segment (start 173.73025 54.75) (end 173.25 54.75) (width 0.2) (layer "F.Cu") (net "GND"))
 (segment (start 168.5 54.75) (end 168.25 54.5) (width 0.2) (layer "F.Cu") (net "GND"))
 (segment (start 167.728436 55.021564) (end 167.728436 55.708052) (width 0.2) (layer "F.Cu") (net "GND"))
 (segment (start 168.25 54.5) (end 167.728436 55.021564) (width 0.2) (layer "F.Cu") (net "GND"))
 (via (at 168.25 68) (size 0.6) (drill 0.3) (layers "F.Cu" "B.Cu") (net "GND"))
 (via (at 174.5 80) (size 0.6) (drill 0.3) (layers "F.Cu" "B.Cu") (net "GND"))
 (via (at 167.728436 55.708052) (size 0.6) (drill 0.3) (layers "F.Cu" "B.Cu") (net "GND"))
 (via (at 187.95 69.420835) (size 0.6) (drill 0.3) (layers "F.Cu" "B.Cu") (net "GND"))
 (via (at 173.25 54.75) (size 0.6) (drill 0.3) (layers "F.Cu" "B.Cu") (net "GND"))
 (via (at 182 54.75) (size 0.6) (drill 0.3) (layers "F.Cu" "B.Cu") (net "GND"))
 (segment (start 187.95 69.420835) (end 187.759165 69.23) (width 0.2) (layer "B.Cu") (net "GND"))
 (segment (start 173.25 54.75) (end 182 54.75) (width 0.2) (layer "B.Cu") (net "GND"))
 (segment (start 185.27 69.23) (end 174.5 80) (width 0.2) (layer "B.Cu") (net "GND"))
 (segment (start 167.58 55.856488) (end 167.58 67.33) (width 0.2) (layer "B.Cu") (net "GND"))
 (segment (start 187.759165 69.23) (end 185.27 69.23) (width 0.2) (layer "B.Cu") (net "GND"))
 (segment (start 167.728436 55.708052) (end 167.58 55.856488) (width 0.2) (layer "B.Cu") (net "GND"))
 (segment (start 167.58 67.33) (end 168.25 68) (width 0.2) (layer "B.Cu") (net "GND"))
 (segment (start 171.31975 41.2545) (end 172.55175 42.4865) (width 0.2) (layer "F.Cu") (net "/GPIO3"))
 (segment (start 175.348096 49.4295) (end 176.02175 50.103154) (width 0.2) (layer "F.Cu") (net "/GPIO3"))
 (segment (start 172.55175 42.4865) (end 172.55175 47.585846) (width 0.2) (layer "F.Cu") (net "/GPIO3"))
 (segment (start 172.55175 47.585846) (end 174.395404 49.4295) (width 0.2) (layer "F.Cu") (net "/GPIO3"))
 (segment (start 176.02175 50.103154) (end 176.02175 51.422172) (width 0.2) (layer "F.Cu") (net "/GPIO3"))
 (segment (start 188.55 63.950422) (end 188.55 86.41) (width 0.2) (layer "F.Cu") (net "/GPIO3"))
 (segment (start 188.55 86.41) (end 183.04 91.92) (width 0.2) (layer "F.Cu") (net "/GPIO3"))
 (segment (start 174.395404 49.4295) (end 175.348096 49.4295) (width 0.2) (layer "F.Cu") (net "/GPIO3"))
 (segment (start 176.02175 51.422172) (end 188.55 63.950422) (width 0.2) (layer "F.Cu") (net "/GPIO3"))
 (segment (start 156.75 54.25) (end 156.324 54.676) (width 0.2) (layer "F.Cu") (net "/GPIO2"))
 (segment (start 174.5 46.25) (end 173.75 47) (width 0.2) (layer "F.Cu") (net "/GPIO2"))
 (segment (start 156.324 85.784) (end 162.46 91.92) (width 0.2) (layer "F.Cu") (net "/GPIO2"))
 (segment (start 156.324 54.676) (end 156.324 85.784) (width 0.2) (layer "F.Cu") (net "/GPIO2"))
 (segment (start 173.85975 41.2545) (end 174.5 41.89475) (width 0.2) (layer "F.Cu") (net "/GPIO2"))
 (segment (start 174.5 41.89475) (end 174.5 46.25) (width 0.2) (layer "F.Cu") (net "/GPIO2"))
 (via (at 173.75 47) (size 0.6) (drill 0.3) (layers "F.Cu" "B.Cu") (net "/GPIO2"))
 (via (at 156.75 54.25) (size 0.6) (drill 0.3) (layers "F.Cu" "B.Cu") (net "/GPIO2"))
 (segment (start 166.5 54.25) (end 156.75 54.25) (width 0.2) (layer "B.Cu") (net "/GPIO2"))
 (segment (start 173.75 47) (end 166.5 54.25) (width 0.2) (layer "B.Cu") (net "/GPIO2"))
 (segment (start 184.348 74.07) (end 187.476346 74.07) (width 0.2) (layer "F.Cu") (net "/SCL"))
 (segment (start 171.27 60.992) (end 184.348 74.07) (width 0.2) (layer "F.Cu") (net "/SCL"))
 (segment (start 162.39975 52.85025) (end 162.39975 58.633142) (width 0.2) (layer "F.Cu") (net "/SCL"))
 (segment (start 187.476346 74.07) (end 188.15 73.396346) (width 0.2) (layer "F.Cu") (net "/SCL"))
 (segment (start 163.608608 59.842) (end 170.12 59.842) (width 0.2) (layer "F.Cu") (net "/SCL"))
 (segment (start 165.25 50) (end 162.39975 52.85025) (width 0.2) (layer "F.Cu") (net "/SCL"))
 (segment (start 188.15 73.396346) (end 188.15 71.53) (width 0.2) (layer "F.Cu") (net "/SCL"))
 (segment (start 188.15 71.53) (end 187 70.38) (width 0.2) (layer "F.Cu") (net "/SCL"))
 (segment (start 168.77975 41.2545) (end 168.77975 44.02975) (width 0.2) (layer "F.Cu") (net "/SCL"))
 (segment (start 168.77975 44.02975) (end 169.5 44.75) (width 0.2) (layer "F.Cu") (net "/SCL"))
 (segment (start 162.39975 58.633142) (end 163.608608 59.842) (width 0.2) (layer "F.Cu") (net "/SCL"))
 (segment (start 170.12 59.842) (end 171.27 60.992) (width 0.2) (layer "F.Cu") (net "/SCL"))
 (via (at 169.5 44.75) (size 0.6) (drill 0.3) (layers "F.Cu" "B.Cu") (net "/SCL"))
 (via (at 165.25 50) (size 0.6) (drill 0.3) (layers "F.Cu" "B.Cu") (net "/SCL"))
 (segment (start 169.5 44.75) (end 169.5 45.75) (width 0.2) (layer "B.Cu") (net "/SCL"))
 (segment (start 169.5 45.75) (end 165.25 50) (width 0.2) (layer "B.Cu") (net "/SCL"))
 (segment (start 178.101108 55.7445) (end 179.778392 55.7445) (width 0.2) (layer "F.Cu") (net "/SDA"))
 (segment (start 166.23975 43.883142) (end 178.101108 55.7445) (width 0.2) (layer "F.Cu") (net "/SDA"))
 (segment (start 185.85 61.816108) (end 185.85 71.77) (width 0.2) (layer "F.Cu") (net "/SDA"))
 (segment (start 166.23975 41.2545) (end 166.23975 43.883142) (width 0.2) (layer "F.Cu") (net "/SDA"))
 (segment (start 185.85 71.77) (end 187 72.92) (width 0.2) (layer "F.Cu") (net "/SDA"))
 (segment (start 179.778392 55.7445) (end 185.85 61.816108) (width 0.2) (layer "F.Cu") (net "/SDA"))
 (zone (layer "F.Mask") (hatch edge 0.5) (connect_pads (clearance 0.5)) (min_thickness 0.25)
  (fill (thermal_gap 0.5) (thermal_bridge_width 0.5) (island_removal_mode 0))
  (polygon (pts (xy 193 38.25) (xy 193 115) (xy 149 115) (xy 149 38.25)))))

